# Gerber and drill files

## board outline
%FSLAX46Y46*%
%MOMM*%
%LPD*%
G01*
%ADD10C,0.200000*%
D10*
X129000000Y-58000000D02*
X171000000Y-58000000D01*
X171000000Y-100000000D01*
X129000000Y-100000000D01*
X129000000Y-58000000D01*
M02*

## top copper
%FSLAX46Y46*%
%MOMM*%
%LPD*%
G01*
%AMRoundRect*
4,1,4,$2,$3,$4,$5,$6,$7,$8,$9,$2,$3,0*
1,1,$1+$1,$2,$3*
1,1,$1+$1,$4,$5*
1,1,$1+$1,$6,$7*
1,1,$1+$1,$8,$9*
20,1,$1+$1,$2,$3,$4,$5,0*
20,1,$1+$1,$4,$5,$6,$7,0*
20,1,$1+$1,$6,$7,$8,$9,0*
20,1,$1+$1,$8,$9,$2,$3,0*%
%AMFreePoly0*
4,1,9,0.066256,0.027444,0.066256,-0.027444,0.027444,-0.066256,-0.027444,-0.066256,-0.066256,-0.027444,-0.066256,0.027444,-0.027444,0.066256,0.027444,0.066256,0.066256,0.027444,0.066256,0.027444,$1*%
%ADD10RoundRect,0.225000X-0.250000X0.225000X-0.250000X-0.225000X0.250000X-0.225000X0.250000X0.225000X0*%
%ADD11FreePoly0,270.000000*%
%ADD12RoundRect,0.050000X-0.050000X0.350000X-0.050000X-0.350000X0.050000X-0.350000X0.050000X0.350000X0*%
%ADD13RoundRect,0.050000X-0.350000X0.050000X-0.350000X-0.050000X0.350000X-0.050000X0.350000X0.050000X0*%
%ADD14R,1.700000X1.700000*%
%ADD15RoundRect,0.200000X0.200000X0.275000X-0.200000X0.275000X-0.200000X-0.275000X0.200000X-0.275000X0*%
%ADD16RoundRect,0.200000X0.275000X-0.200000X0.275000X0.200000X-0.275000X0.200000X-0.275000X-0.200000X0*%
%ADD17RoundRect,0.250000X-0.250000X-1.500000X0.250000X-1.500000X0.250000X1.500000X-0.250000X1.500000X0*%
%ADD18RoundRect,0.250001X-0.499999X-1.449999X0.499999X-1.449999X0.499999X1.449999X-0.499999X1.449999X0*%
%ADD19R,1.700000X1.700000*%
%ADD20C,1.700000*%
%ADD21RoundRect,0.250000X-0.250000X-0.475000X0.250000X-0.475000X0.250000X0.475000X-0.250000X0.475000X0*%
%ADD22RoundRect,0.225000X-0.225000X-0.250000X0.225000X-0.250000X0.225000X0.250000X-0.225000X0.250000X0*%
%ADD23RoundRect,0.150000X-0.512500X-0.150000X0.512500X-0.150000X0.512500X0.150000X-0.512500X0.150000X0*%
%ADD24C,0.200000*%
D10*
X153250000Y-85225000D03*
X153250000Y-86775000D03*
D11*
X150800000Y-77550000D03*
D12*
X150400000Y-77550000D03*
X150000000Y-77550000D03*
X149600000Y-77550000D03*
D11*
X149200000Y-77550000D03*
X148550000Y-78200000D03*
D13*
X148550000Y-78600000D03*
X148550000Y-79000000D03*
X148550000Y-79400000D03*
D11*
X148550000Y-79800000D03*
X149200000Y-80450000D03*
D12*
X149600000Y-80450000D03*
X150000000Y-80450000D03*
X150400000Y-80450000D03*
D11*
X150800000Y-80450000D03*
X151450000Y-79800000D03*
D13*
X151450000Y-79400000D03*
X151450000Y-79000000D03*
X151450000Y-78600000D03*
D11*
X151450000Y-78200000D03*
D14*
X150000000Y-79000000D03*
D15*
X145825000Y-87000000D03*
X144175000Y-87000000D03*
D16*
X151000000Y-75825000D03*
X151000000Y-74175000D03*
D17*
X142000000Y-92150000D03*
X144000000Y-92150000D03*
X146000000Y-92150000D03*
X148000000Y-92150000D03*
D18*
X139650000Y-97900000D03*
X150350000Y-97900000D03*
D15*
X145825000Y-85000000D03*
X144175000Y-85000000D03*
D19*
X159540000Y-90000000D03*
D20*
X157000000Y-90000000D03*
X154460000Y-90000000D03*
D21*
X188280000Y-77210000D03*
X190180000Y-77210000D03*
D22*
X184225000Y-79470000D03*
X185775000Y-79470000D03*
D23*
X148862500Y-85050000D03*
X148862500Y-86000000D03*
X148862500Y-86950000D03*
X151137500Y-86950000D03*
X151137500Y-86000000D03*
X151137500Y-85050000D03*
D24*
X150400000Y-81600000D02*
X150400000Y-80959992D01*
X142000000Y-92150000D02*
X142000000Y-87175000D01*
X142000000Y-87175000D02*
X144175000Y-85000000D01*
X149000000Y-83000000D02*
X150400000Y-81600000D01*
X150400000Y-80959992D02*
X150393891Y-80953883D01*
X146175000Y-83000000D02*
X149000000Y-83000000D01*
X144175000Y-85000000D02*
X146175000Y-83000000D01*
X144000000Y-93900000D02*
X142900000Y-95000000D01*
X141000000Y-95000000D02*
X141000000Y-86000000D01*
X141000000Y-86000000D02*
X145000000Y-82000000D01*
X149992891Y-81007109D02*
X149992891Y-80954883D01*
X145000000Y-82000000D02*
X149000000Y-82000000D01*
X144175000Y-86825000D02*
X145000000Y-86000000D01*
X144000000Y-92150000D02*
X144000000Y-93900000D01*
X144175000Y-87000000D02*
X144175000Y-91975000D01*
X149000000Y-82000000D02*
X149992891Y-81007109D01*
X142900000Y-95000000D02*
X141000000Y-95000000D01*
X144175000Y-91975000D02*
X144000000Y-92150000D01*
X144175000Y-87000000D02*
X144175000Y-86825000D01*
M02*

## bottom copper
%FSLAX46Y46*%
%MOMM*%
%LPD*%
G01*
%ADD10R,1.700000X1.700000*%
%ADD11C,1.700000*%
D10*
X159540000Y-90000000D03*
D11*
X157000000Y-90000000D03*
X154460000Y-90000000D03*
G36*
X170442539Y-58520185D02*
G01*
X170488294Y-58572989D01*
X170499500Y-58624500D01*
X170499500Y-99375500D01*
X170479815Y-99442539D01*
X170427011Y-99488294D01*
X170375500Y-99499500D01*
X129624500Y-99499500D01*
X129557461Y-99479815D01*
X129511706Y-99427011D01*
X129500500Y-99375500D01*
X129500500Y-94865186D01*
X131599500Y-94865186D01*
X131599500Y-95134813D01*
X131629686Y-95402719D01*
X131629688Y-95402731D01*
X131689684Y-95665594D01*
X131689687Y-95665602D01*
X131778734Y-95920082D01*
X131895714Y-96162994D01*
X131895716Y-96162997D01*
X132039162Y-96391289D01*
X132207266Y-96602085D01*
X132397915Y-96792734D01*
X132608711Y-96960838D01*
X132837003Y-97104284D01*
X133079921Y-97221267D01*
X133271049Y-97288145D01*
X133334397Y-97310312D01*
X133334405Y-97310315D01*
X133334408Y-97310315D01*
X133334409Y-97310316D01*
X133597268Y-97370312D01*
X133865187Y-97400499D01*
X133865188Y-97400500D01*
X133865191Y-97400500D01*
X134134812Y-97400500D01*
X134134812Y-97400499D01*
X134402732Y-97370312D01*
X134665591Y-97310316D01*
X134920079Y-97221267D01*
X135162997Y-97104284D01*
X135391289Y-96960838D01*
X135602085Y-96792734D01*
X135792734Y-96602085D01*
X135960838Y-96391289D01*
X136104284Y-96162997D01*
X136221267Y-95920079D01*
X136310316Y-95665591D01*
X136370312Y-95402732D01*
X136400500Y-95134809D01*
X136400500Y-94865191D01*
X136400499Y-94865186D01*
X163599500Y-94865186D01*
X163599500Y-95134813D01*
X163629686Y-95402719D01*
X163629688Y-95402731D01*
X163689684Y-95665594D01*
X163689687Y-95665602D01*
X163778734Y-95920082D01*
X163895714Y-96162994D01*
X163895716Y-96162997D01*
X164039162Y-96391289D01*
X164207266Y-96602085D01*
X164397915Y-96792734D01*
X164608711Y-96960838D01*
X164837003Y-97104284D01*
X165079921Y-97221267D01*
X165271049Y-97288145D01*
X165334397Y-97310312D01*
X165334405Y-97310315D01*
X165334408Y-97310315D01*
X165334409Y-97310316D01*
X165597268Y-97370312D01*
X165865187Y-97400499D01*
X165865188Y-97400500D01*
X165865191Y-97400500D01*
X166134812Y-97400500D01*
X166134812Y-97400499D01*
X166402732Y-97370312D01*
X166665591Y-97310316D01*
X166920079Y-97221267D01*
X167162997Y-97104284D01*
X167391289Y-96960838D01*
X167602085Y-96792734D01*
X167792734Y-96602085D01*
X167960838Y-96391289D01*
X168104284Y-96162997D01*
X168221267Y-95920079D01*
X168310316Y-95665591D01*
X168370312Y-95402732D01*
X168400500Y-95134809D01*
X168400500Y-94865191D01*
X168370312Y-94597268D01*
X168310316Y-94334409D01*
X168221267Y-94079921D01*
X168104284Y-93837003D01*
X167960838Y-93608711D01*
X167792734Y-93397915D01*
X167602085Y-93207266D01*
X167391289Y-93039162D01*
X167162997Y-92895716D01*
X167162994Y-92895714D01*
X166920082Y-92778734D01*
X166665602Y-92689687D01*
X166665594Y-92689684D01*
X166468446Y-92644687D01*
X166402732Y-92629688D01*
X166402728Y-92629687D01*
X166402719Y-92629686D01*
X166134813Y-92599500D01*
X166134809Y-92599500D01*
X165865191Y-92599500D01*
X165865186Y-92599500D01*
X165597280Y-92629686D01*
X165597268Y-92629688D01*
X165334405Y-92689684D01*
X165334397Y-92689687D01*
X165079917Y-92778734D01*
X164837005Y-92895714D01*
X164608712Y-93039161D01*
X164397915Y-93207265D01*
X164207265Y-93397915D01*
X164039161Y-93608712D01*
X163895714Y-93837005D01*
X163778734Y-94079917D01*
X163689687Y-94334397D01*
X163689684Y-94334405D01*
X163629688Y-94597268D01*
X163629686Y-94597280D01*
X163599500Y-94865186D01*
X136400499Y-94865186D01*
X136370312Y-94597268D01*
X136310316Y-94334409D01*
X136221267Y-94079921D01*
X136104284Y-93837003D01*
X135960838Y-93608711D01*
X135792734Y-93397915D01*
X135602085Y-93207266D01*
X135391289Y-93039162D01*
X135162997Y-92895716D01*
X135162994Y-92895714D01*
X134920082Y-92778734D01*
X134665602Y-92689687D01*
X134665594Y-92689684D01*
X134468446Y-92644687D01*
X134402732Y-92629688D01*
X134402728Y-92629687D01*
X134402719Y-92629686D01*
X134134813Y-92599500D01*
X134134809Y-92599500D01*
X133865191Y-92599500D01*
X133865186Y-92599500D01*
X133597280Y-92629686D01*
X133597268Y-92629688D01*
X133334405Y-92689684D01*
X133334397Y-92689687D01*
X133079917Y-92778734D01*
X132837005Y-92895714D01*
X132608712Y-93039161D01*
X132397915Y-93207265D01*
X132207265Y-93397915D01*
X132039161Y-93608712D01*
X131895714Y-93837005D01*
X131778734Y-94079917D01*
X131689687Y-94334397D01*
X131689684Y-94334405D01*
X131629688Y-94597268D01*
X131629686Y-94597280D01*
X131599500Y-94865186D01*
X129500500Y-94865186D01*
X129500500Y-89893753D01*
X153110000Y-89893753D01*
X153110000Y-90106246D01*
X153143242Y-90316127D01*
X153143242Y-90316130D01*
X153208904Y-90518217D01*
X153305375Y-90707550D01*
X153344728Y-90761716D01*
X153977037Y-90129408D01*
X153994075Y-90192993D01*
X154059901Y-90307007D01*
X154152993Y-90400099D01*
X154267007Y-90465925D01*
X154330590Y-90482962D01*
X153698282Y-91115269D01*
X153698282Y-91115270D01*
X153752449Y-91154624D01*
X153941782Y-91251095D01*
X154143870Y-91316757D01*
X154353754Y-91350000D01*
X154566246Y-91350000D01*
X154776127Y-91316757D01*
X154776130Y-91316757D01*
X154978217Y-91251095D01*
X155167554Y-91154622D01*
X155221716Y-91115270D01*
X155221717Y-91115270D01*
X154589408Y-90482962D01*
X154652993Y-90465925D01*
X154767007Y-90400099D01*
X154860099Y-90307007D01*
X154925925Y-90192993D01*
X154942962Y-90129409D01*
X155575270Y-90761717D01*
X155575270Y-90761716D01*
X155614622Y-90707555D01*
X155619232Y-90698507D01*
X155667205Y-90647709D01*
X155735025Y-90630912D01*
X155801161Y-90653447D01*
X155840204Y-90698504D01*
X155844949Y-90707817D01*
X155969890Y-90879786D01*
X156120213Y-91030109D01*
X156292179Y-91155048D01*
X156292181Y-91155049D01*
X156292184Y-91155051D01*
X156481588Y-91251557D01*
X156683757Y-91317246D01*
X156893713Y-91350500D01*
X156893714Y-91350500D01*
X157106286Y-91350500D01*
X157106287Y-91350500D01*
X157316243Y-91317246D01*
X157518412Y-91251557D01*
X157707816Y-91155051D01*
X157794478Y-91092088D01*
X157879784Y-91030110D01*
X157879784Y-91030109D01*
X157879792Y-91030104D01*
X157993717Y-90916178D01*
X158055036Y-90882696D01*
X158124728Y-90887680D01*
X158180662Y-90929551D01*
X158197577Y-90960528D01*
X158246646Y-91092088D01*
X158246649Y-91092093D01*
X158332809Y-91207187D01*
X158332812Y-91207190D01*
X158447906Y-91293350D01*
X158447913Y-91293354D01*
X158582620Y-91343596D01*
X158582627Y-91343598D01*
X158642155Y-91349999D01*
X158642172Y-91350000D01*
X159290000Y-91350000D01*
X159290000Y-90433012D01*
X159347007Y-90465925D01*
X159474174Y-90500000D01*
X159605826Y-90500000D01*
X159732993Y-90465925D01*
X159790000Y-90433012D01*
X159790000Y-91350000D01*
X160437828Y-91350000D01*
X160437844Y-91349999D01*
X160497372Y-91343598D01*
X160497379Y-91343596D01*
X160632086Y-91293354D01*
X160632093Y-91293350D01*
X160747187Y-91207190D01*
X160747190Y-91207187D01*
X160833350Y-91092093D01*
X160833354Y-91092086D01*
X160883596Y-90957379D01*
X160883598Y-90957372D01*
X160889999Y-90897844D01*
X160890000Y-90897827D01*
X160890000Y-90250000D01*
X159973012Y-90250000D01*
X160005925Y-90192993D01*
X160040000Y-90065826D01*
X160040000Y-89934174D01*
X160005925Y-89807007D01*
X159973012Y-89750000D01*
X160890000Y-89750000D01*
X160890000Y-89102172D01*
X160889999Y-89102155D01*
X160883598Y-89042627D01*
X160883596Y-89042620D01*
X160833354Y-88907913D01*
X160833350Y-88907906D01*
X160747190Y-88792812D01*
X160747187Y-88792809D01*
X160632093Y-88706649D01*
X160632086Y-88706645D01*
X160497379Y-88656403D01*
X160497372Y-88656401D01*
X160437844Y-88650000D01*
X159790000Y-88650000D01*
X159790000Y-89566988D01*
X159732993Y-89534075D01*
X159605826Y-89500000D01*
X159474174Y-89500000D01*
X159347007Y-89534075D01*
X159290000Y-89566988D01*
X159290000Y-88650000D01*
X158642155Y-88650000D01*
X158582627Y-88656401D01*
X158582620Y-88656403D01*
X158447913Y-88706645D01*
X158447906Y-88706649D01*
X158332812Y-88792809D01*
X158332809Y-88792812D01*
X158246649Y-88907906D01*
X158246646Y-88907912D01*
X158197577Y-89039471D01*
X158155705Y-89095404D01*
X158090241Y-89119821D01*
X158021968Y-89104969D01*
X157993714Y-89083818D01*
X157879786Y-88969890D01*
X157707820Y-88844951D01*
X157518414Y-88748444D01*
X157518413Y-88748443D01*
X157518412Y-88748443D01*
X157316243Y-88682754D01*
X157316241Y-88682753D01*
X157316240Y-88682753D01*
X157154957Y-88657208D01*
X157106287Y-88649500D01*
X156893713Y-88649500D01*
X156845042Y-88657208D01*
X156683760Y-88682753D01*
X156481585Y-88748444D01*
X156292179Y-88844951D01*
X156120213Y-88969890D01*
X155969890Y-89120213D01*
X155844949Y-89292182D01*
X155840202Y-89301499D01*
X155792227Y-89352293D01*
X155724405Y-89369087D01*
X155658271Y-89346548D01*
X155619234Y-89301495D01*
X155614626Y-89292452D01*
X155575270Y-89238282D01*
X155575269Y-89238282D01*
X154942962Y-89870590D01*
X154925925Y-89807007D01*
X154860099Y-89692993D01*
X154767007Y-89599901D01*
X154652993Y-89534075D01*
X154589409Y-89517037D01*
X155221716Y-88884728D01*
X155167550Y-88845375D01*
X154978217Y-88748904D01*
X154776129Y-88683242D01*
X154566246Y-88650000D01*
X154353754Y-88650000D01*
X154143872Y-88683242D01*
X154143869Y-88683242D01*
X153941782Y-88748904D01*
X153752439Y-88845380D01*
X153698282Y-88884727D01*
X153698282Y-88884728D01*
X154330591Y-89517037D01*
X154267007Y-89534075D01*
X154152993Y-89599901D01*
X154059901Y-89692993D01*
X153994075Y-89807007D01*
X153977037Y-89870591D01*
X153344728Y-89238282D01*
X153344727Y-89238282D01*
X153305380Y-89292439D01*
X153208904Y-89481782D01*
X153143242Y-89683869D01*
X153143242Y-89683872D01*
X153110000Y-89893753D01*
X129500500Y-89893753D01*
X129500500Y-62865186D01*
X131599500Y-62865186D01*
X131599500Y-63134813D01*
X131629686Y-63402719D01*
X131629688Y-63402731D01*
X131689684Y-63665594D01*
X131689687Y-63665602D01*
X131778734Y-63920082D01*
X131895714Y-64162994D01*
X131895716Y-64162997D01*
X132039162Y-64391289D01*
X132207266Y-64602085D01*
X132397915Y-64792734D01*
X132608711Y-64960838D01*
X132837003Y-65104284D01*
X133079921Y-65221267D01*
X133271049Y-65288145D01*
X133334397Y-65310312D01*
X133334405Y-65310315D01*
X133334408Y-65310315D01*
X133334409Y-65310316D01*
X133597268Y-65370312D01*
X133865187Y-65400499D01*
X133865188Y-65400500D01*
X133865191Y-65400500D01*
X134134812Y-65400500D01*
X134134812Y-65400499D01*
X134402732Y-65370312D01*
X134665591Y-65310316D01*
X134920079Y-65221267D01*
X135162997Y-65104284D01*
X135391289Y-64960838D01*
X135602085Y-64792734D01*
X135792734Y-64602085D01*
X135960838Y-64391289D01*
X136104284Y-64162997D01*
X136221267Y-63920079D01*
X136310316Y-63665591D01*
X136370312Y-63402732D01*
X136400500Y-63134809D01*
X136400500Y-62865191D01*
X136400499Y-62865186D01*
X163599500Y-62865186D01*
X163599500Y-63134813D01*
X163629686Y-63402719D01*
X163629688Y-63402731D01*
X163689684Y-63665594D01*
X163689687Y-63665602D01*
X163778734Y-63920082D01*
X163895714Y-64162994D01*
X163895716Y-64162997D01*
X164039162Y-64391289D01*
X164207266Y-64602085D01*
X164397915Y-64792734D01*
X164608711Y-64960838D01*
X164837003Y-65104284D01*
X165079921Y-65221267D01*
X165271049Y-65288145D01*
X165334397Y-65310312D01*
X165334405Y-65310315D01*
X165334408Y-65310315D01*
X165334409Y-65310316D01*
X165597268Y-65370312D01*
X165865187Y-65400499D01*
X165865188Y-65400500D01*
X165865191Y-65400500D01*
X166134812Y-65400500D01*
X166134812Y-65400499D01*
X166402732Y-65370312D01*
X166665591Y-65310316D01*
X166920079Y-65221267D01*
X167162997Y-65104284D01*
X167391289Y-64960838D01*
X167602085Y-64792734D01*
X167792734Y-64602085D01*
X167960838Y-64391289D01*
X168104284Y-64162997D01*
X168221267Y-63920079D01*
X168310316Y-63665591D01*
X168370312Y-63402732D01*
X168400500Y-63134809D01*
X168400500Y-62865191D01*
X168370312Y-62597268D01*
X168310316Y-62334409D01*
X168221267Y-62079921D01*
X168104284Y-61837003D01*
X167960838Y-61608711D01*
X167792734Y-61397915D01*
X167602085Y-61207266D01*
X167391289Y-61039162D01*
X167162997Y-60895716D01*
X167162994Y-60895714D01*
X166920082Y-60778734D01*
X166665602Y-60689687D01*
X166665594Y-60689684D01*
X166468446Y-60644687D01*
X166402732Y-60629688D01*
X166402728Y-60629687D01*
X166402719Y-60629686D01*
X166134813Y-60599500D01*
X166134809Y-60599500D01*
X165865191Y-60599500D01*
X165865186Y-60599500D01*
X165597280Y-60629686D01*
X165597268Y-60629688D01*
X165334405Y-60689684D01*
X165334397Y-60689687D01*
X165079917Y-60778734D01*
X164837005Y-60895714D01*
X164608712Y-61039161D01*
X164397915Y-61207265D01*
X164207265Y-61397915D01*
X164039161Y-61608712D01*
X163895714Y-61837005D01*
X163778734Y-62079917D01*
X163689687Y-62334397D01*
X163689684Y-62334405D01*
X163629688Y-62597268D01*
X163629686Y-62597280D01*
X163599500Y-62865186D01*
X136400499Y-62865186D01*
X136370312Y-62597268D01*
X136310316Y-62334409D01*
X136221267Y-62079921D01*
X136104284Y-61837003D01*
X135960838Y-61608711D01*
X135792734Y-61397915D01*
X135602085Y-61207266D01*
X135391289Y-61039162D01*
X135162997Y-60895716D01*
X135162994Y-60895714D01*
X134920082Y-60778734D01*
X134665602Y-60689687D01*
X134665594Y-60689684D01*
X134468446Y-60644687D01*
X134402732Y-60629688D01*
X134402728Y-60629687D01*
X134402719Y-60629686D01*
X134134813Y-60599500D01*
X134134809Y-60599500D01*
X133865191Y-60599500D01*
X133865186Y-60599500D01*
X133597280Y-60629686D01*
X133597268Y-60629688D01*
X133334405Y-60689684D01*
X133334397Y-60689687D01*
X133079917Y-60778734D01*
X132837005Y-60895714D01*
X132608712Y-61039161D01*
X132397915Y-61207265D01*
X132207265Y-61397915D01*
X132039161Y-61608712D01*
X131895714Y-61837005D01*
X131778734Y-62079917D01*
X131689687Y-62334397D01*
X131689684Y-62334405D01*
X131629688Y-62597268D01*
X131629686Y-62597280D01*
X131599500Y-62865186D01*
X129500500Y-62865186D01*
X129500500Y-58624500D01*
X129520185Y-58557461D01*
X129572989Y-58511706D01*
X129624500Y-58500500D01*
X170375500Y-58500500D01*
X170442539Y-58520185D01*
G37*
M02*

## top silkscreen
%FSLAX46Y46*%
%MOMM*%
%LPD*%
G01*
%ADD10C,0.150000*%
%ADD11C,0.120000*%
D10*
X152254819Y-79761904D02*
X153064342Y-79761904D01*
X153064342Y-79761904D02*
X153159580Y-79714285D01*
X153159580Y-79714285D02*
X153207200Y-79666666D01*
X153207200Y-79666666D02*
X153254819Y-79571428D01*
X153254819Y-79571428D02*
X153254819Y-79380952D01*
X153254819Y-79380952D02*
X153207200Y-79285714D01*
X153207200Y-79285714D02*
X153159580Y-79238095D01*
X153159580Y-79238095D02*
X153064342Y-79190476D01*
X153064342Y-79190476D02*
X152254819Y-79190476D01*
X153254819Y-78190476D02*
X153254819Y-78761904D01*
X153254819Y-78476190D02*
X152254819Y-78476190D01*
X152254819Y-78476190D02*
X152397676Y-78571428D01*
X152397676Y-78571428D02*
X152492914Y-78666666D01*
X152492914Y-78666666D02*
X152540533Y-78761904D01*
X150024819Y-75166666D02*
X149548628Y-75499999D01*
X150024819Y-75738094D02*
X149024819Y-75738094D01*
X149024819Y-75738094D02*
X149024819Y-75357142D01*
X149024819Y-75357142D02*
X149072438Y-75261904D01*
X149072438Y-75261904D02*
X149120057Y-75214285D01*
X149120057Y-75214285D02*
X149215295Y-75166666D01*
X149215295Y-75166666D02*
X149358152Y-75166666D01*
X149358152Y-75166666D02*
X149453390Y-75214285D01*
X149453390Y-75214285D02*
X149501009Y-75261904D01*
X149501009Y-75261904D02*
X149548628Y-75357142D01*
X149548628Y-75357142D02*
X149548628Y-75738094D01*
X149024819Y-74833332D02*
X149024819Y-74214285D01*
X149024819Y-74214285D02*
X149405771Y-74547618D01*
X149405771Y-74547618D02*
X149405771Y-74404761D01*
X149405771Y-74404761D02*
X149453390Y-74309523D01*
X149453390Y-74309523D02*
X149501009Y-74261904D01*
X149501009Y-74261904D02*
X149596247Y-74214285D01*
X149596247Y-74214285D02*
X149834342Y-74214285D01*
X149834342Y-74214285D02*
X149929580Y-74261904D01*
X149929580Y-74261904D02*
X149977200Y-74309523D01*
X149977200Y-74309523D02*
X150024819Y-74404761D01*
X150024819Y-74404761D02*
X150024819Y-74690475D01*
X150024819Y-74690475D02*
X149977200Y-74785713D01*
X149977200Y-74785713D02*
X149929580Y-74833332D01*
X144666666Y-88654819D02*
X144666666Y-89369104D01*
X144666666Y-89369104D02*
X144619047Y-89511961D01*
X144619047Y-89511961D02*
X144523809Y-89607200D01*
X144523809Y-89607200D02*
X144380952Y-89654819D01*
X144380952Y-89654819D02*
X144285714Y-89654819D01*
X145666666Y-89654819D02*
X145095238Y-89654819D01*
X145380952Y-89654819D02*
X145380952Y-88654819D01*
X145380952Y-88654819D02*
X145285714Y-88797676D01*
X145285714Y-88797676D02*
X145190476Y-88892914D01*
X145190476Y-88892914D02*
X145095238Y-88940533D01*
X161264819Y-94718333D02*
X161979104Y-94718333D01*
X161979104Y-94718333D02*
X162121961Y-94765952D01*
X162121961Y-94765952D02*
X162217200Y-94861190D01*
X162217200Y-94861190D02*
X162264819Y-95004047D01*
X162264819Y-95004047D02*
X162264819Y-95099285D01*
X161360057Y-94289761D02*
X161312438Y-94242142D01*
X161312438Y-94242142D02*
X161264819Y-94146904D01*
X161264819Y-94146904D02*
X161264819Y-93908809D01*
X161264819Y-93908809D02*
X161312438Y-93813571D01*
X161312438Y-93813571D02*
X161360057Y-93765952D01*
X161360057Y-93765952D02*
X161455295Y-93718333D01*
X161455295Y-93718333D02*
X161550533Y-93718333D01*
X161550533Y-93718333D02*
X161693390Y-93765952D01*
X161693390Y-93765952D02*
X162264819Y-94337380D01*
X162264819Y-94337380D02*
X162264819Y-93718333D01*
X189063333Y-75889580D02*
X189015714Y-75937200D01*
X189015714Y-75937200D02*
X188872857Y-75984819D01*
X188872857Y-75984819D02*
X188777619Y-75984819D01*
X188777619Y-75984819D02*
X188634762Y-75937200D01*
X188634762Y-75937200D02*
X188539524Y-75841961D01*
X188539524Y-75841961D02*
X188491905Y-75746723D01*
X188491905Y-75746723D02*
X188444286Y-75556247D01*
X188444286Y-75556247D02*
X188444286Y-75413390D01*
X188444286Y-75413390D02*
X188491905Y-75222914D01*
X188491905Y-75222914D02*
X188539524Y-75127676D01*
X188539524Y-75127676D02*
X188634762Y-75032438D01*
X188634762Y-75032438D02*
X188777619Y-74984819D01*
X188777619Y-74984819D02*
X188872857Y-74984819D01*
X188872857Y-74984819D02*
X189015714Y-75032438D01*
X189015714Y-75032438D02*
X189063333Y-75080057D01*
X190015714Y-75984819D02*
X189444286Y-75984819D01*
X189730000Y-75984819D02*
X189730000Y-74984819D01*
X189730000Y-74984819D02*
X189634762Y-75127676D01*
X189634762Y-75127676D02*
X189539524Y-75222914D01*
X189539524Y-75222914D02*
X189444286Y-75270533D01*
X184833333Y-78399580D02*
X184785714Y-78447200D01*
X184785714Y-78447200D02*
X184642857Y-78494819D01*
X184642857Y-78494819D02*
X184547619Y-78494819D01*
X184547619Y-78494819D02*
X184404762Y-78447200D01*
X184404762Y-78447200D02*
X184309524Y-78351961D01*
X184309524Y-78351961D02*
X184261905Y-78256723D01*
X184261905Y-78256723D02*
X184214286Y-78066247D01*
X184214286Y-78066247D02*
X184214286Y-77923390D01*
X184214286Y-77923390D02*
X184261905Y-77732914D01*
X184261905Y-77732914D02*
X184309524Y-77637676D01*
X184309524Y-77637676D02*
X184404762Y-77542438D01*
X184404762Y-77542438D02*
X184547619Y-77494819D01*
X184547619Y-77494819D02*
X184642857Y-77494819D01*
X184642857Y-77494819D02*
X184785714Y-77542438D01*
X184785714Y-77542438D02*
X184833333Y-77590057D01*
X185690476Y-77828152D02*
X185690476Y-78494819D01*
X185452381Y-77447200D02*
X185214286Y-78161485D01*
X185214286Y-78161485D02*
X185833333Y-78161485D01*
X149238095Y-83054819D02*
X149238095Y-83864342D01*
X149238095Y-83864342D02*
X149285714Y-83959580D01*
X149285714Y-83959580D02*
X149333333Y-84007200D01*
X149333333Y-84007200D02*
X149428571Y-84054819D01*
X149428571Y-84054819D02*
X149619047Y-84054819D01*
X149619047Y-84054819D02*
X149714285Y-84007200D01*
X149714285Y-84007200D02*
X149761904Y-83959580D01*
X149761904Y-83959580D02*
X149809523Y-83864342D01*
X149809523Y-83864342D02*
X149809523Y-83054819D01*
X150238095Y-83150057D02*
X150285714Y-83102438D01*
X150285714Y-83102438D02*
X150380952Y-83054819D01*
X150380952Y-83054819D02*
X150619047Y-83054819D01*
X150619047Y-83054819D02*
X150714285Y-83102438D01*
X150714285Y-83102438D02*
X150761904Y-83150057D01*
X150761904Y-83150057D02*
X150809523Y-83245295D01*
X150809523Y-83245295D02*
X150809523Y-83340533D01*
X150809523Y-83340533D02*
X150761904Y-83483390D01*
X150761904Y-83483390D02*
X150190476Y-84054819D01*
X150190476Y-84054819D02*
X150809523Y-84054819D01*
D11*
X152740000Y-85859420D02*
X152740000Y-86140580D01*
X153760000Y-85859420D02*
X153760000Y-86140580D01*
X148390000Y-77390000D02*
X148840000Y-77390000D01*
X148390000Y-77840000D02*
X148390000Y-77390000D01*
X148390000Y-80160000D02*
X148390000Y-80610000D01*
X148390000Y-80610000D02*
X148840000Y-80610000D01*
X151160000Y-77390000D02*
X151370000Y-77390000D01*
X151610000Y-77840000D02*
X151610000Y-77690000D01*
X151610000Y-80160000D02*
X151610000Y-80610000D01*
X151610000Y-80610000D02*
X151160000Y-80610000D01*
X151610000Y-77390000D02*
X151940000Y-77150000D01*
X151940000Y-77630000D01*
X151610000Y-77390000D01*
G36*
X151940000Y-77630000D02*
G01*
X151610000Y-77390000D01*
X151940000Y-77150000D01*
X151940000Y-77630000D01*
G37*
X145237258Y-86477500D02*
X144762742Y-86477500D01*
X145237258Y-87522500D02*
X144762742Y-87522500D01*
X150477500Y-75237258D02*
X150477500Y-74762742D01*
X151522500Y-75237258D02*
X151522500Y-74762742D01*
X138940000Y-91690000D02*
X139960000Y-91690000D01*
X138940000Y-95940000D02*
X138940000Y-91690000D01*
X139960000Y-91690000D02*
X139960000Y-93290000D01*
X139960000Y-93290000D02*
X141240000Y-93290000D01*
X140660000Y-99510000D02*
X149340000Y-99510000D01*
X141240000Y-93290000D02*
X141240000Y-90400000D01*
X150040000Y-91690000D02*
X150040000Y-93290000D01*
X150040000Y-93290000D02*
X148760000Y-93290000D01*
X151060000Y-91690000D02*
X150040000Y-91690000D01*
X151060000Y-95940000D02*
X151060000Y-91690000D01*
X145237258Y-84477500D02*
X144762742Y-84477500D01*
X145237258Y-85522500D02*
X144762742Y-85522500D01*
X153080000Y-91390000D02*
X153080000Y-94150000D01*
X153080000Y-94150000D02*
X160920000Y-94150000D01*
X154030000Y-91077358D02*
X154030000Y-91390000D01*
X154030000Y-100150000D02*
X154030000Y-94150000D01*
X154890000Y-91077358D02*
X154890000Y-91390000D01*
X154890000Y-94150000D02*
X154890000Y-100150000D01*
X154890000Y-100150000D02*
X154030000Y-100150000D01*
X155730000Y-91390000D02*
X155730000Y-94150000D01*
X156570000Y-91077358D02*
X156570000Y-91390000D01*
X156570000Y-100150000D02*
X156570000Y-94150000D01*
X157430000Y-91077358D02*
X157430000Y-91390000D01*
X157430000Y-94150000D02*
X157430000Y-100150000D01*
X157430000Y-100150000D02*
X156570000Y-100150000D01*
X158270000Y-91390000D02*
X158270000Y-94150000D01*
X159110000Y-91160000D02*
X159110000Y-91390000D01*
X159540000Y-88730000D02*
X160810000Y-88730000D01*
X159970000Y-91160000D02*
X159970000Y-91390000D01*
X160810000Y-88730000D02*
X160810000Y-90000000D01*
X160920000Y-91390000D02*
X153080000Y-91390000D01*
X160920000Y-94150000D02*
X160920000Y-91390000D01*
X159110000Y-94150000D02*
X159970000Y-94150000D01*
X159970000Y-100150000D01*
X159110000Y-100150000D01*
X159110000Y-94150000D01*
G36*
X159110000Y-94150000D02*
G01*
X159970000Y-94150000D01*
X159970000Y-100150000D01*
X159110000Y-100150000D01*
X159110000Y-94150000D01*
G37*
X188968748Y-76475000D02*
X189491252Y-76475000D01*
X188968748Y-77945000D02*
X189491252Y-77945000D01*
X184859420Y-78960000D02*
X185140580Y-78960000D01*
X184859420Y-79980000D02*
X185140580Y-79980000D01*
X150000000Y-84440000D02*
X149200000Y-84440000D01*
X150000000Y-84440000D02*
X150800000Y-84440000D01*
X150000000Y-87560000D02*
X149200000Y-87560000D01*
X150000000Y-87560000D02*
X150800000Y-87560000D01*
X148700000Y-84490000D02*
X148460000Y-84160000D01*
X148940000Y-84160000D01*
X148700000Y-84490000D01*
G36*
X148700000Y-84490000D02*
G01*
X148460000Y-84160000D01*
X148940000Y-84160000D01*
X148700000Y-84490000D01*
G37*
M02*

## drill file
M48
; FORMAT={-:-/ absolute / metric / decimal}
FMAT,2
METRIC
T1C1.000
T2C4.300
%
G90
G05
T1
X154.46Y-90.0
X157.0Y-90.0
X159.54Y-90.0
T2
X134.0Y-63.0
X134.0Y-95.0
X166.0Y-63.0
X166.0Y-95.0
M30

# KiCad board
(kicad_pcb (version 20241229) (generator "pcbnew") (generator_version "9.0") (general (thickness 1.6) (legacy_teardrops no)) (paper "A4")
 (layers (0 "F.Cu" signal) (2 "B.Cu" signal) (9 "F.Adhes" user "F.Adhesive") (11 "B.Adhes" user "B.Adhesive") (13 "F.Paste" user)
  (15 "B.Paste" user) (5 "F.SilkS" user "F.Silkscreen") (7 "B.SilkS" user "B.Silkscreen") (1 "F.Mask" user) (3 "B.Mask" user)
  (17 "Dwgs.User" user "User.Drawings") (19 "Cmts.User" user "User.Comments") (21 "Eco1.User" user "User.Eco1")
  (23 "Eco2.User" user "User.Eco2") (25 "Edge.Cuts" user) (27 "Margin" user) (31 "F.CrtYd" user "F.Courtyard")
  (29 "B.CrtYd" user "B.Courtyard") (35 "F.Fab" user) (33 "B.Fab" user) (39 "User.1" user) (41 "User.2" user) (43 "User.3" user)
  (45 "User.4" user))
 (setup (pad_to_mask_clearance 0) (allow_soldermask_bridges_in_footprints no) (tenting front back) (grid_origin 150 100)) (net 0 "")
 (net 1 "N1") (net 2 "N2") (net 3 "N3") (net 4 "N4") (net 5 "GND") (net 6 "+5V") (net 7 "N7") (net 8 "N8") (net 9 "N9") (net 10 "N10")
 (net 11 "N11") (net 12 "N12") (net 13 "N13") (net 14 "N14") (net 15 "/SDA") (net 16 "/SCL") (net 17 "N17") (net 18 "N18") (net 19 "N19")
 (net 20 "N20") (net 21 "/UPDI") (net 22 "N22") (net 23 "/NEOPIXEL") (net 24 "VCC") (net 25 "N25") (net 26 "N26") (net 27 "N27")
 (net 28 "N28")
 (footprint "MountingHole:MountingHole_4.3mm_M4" (layer "F.Cu") (at 134 63)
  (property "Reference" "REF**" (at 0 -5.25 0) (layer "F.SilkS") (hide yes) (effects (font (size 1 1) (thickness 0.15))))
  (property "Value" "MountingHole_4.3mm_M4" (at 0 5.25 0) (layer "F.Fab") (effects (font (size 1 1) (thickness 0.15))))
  (pad "" np_thru_hole circle (at 0 0) (size 4.3 4.3) (drill 4.3) (layers "*.Cu" "*.Mask")))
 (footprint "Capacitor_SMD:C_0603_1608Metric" (layer "F.Cu") (at 153.25 86 -90)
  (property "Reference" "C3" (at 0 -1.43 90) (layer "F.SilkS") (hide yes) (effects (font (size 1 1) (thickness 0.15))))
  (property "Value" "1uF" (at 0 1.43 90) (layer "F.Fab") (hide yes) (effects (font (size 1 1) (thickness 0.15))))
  (fp_line (start -0.14058 0.51) (end 0.14058 0.51) (stroke (width 0.12) (type solid)) (layer "F.SilkS"))
  (fp_line (start -0.14058 -0.51) (end 0.14058 -0.51) (stroke (width 0.12) (type solid)) (layer "F.SilkS"))
  (pad "1" smd roundrect (at -0.775 0 270) (size 0.9 0.95) (layers "F.Cu" "F.Mask" "F.Paste") (roundrect_rratio 0.25) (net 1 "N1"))
  (pad "2" smd roundrect (at 0.775 0 270) (size 0.9 0.95) (layers "F.Cu" "F.Mask" "F.Paste") (roundrect_rratio 0.25) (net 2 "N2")))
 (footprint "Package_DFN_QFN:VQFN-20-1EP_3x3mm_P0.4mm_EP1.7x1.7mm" (layer "F.Cu") (at 150 79 -90)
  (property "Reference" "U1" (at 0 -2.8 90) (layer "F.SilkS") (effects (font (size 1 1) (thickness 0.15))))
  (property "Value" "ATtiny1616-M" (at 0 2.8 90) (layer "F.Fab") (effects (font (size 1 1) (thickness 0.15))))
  (fp_line (start -1.61 1.61) (end -1.61 1.16) (stroke (width 0.12) (type solid)) (layer "F.SilkS"))
  (fp_line (start -1.16 1.61) (end -1.61 1.61) (stroke (width 0.12) (type solid)) (layer "F.SilkS"))
  (fp_line (start 1.16 1.61) (end 1.61 1.61) (stroke (width 0.12) (type solid)) (layer "F.SilkS"))
  (fp_line (start 1.61 1.61) (end 1.61 1.16) (stroke (width 0.12) (type solid)) (layer "F.SilkS"))
  (fp_line (start -1.61 -1.16) (end -1.61 -1.37) (stroke (width 0.12) (type solid)) (layer "F.SilkS"))
  (fp_line (start -1.16 -1.61) (end -1.31 -1.61) (stroke (width 0.12) (type solid)) (layer "F.SilkS"))
  (fp_line (start 1.16 -1.61) (end 1.61 -1.61) (stroke (width 0.12) (type solid)) (layer "F.SilkS"))
  (fp_line (start 1.61 -1.61) (end 1.61 -1.16) (stroke (width 0.12) (type solid)) (layer "F.SilkS"))
  (fp_poly (pts (xy -1.61 -1.61) (xy -1.85 -1.94) (xy -1.37 -1.94)) (stroke (width 0.12) (type solid)) (fill yes) (layer "F.SilkS"))
  (pad "" smd roundrect (at -0.425 -0.425 270) (size 0.69 0.69) (layers "F.Paste") (roundrect_rratio 0.25))
  (pad "" smd roundrect (at -0.425 0.425 270) (size 0.69 0.69) (layers "F.Paste") (roundrect_rratio 0.25))
  (pad "" smd roundrect (at 0.425 -0.425 270) (size 0.69 0.69) (layers "F.Paste") (roundrect_rratio 0.25))
  (pad "" smd roundrect (at 0.425 0.425 270) (size 0.69 0.69) (layers "F.Paste") (roundrect_rratio 0.25))
  (pad "1" smd custom (at -1.45 -0.8 270) (size 0.143431 0.143431) (layers "F.Cu" "F.Mask" "F.Paste") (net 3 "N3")
   (options (clearance outline) (anchor circle)) (primitives))
  (pad "2" smd roundrect (at -1.45 -0.4 270) (size 0.8 0.2) (layers "F.Cu" "F.Mask" "F.Paste") (roundrect_rratio 0.25) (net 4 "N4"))
  (pad "3" smd roundrect (at -1.45 0 270) (size 0.8 0.2) (layers "F.Cu" "F.Mask" "F.Paste") (roundrect_rratio 0.25) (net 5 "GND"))
  (pad "4" smd roundrect (at -1.45 0.4 270) (size 0.8 0.2) (layers "F.Cu" "F.Mask" "F.Paste") (roundrect_rratio 0.25) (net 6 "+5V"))
  (pad "5" smd custom (at -1.45 0.8 270) (size 0.143431 0.143431) (layers "F.Cu" "F.Mask" "F.Paste") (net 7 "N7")
   (options (clearance outline) (anchor circle)) (primitives))
  (pad "6" smd custom (at -0.8 1.45 270) (size 0.143431 0.143431) (layers "F.Cu" "F.Mask" "F.Paste") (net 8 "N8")
   (options (clearance outline) (anchor circle)) (primitives))
  (pad "7" smd roundrect (at -0.4 1.45 270) (size 0.2 0.8) (layers "F.Cu" "F.Mask" "F.Paste") (roundrect_rratio 0.25) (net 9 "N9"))
  (pad "8" smd roundrect (at 0 1.45 270) (size 0.2 0.8) (layers "F.Cu" "F.Mask" "F.Paste") (roundrect_rratio 0.25) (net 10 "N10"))
  (pad "9" smd roundrect (at 0.4 1.45 270) (size 0.2 0.8) (layers "F.Cu" "F.Mask" "F.Paste") (roundrect_rratio 0.25) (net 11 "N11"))
  (pad "10" smd custom (at 0.8 1.45 270) (size 0.143431 0.143431) (layers "F.Cu" "F.Mask" "F.Paste") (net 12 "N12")
   (options (clearance outline) (anchor circle)) (primitives))
  (pad "11" smd custom (at 1.45 0.8 270) (size 0.143431 0.143431) (layers "F.Cu" "F.Mask" "F.Paste") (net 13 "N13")
   (options (clearance outline) (anchor circle)) (primitives))
  (pad "12" smd roundrect (at 1.45 0.4 270) (size 0.8 0.2) (layers "F.Cu" "F.Mask" "F.Paste") (roundrect_rratio 0.25) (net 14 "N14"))
  (pad "13" smd roundrect (at 1.45 0 270) (size 0.8 0.2) (layers "F.Cu" "F.Mask" "F.Paste") (roundrect_rratio 0.25) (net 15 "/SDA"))
  (pad "14" smd roundrect (at 1.45 -0.4 270) (size 0.8 0.2) (layers "F.Cu" "F.Mask" "F.Paste") (roundrect_rratio 0.25) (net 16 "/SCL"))
  (pad "15" smd custom (at 1.45 -0.8 270) (size 0.143431 0.143431) (layers "F.Cu" "F.Mask" "F.Paste") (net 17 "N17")
   (options (clearance outline) (anchor circle)) (primitives))
  (pad "16" smd custom (at 0.8 -1.45 270) (size 0.143431 0.143431) (layers "F.Cu" "F.Mask" "F.Paste") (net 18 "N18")
   (options (clearance outline) (anchor circle)) (primitives))
  (pad "17" smd roundrect (at 0.4 -1.45 270) (size 0.2 0.8) (layers "F.Cu" "F.Mask" "F.Paste") (roundrect_rratio 0.25) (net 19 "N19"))
  (pad "18" smd roundrect (at 0 -1.45 270) (size 0.2 0.8) (layers "F.Cu" "F.Mask" "F.Paste") (roundrect_rratio 0.25) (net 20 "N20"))
  (pad "19" smd roundrect (at -0.4 -1.45 270) (size 0.2 0.8) (layers "F.Cu" "F.Mask" "F.Paste") (roundrect_rratio 0.25) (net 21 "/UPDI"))
  (pad "20" smd custom (at -0.8 -1.45 270) (size 0.143431 0.143431) (layers "F.Cu" "F.Mask" "F.Paste") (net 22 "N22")
   (options (clearance outline) (anchor circle)) (primitives))
  (pad "21" smd rect (at 0 0 270) (size 1.7 1.7) (layers "F.Cu" "F.Mask") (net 5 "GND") (zone_connect 2)))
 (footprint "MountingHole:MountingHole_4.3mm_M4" (layer "F.Cu") (at 166 63)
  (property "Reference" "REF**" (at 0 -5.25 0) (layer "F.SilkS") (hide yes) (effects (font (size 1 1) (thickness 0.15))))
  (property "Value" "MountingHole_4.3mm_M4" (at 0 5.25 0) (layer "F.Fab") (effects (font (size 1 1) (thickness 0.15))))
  (pad "" np_thru_hole circle (at 0 0) (size 4.3 4.3) (drill 4.3) (layers "*.Cu" "*.Mask")))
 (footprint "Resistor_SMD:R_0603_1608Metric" (layer "F.Cu") (at 145 87 180)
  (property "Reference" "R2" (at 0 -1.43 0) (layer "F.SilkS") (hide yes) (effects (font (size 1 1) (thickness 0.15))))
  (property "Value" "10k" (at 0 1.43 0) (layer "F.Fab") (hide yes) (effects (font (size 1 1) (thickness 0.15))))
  (fp_line (start -0.237258 0.5225) (end 0.237258 0.5225) (stroke (width 0.12) (type solid)) (layer "F.SilkS"))
  (fp_line (start -0.237258 -0.5225) (end 0.237258 -0.5225) (stroke (width 0.12) (type solid)) (layer "F.SilkS"))
  (pad "1" smd roundrect (at -0.825 0 180) (size 0.8 0.95) (layers "F.Cu" "F.Mask" "F.Paste") (roundrect_rratio 0.25) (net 6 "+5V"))
  (pad "2" smd roundrect (at 0.825 0 180) (size 0.8 0.95) (layers "F.Cu" "F.Mask" "F.Paste") (roundrect_rratio 0.25) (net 15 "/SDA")))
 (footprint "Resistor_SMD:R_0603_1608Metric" (layer "F.Cu") (at 151 75 90)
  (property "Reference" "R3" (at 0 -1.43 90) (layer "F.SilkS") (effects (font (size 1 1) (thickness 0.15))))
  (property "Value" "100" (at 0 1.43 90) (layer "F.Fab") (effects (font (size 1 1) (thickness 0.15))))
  (fp_line (start -0.237258 -0.5225) (end 0.237258 -0.5225) (stroke (width 0.12) (type solid)) (layer "F.SilkS"))
  (fp_line (start -0.237258 0.5225) (end 0.237258 0.5225) (stroke (width 0.12) (type solid)) (layer "F.SilkS"))
  (pad "1" smd roundrect (at -0.825 0 90) (size 0.8 0.95) (layers "F.Cu" "F.Mask" "F.Paste") (roundrect_rratio 0.25) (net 3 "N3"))
  (pad "2" smd roundrect (at 0.825 0 90) (size 0.8 0.95) (layers "F.Cu" "F.Mask" "F.Paste") (roundrect_rratio 0.25) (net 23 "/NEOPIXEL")))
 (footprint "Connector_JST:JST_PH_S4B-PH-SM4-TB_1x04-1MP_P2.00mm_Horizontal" (layer "F.Cu") (at 145 95)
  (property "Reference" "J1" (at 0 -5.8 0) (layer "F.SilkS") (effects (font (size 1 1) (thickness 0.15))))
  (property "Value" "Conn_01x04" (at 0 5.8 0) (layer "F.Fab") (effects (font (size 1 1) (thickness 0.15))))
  (fp_line (start -6.06 -3.31) (end -5.04 -3.31) (stroke (width 0.12) (type solid)) (layer "F.SilkS"))
  (fp_line (start -6.06 0.94) (end -6.06 -3.31) (stroke (width 0.12) (type solid)) (layer "F.SilkS"))
  (fp_line (start -5.04 -3.31) (end -5.04 -1.71) (stroke (width 0.12) (type solid)) (layer "F.SilkS"))
  (fp_line (start -5.04 -1.71) (end -3.76 -1.71) (stroke (width 0.12) (type solid)) (layer "F.SilkS"))
  (fp_line (start -4.34 4.51) (end 4.34 4.51) (stroke (width 0.12) (type solid)) (layer "F.SilkS"))
  (fp_line (start -3.76 -1.71) (end -3.76 -4.6) (stroke (width 0.12) (type solid)) (layer "F.SilkS"))
  (fp_line (start 5.04 -3.31) (end 5.04 -1.71) (stroke (width 0.12) (type solid)) (layer "F.SilkS"))
  (fp_line (start 5.04 -1.71) (end 3.76 -1.71) (stroke (width 0.12) (type solid)) (layer "F.SilkS"))
  (fp_line (start 6.06 -3.31) (end 5.04 -3.31) (stroke (width 0.12) (type solid)) (layer "F.SilkS"))
  (fp_line (start 6.06 0.94) (end 6.06 -3.31) (stroke (width 0.12) (type solid)) (layer "F.SilkS"))
  (pad "1" smd roundrect (at -3 -2.85) (size 1 3.5) (layers "F.Cu" "F.Mask" "F.Paste") (roundrect_rratio 0.25) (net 16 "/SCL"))
  (pad "2" smd roundrect (at -1 -2.85) (size 1 3.5) (layers "F.Cu" "F.Mask" "F.Paste") (roundrect_rratio 0.25) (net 15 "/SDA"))
  (pad "3" smd roundrect (at 1 -2.85) (size 1 3.5) (layers "F.Cu" "F.Mask" "F.Paste") (roundrect_rratio 0.25) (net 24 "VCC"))
  (pad "4" smd roundrect (at 3 -2.85) (size 1 3.5) (layers "F.Cu" "F.Mask" "F.Paste") (roundrect_rratio 0.25) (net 5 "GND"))
  (pad "MP" smd roundrect (at -5.35 2.9) (size 1.5 3.4) (layers "F.Cu" "F.Mask" "F.Paste") (roundrect_rratio 0.166667))
  (pad "MP" smd roundrect (at 5.35 2.9) (size 1.5 3.4) (layers "F.Cu" "F.Mask" "F.Paste") (roundrect_rratio 0.166667)))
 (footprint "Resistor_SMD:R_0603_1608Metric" (layer "F.Cu") (at 145 85 180)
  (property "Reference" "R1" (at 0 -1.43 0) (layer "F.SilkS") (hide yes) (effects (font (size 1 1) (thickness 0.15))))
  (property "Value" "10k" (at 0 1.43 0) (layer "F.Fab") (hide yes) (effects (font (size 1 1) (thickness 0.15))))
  (fp_line (start -0.237258 0.5225) (end 0.237258 0.5225) (stroke (width 0.12) (type solid)) (layer "F.SilkS"))
  (fp_line (start -0.237258 -0.5225) (end 0.237258 -0.5225) (stroke (width 0.12) (type solid)) (layer "F.SilkS"))
  (pad "1" smd roundrect (at -0.825 0 180) (size 0.8 0.95) (layers "F.Cu" "F.Mask" "F.Paste") (roundrect_rratio 0.25) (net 6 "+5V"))
  (pad "2" smd roundrect (at 0.825 0 180) (size 0.8 0.95) (layers "F.Cu" "F.Mask" "F.Paste") (roundrect_rratio 0.25) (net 16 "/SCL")))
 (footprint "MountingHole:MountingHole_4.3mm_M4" (layer "F.Cu") (at 166 95)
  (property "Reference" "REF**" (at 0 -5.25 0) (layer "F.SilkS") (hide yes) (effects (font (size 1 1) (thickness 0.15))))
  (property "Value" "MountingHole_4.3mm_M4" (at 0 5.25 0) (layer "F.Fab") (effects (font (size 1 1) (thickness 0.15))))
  (pad "" np_thru_hole circle (at 0 0) (size 4.3 4.3) (drill 4.3) (layers "*.Cu" "*.Mask")))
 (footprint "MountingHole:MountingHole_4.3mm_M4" (layer "F.Cu") (at 134 95)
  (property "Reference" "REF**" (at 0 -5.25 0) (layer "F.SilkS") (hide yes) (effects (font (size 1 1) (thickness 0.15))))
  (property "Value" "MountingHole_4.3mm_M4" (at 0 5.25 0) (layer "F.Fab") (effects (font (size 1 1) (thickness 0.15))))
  (pad "" np_thru_hole circle (at 0 0) (size 4.3 4.3) (drill 4.3) (layers "*.Cu" "*.Mask")))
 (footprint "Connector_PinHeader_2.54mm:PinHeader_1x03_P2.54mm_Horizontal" (layer "F.Cu") (at 159.54 90 -90)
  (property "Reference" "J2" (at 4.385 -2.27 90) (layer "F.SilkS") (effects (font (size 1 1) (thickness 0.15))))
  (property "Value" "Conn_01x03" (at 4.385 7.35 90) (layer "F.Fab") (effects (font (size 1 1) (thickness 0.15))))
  (fp_line (start 1.39 6.46) (end 4.15 6.46) (stroke (width 0.12) (type solid)) (layer "F.SilkS"))
  (fp_line (start 4.15 6.46) (end 4.15 -1.38) (stroke (width 0.12) (type solid)) (layer "F.SilkS"))
  (fp_line (start 1.077358 5.51) (end 1.39 5.51) (stroke (width 0.12) (type solid)) (layer "F.SilkS"))
  (fp_line (start 10.15 5.51) (end 4.15 5.51) (stroke (width 0.12) (type solid)) (layer "F.SilkS"))
  (fp_line (start 1.077358 4.65) (end 1.39 4.65) (stroke (width 0.12) (type solid)) (layer "F.SilkS"))
  (fp_line (start 4.15 4.65) (end 10.15 4.65) (stroke (width 0.12) (type solid)) (layer "F.SilkS"))
  (fp_line (start 10.15 4.65) (end 10.15 5.51) (stroke (width 0.12) (type solid)) (layer "F.SilkS"))
  (fp_line (start 1.39 3.81) (end 4.15 3.81) (stroke (width 0.12) (type solid)) (layer "F.SilkS"))
  (fp_line (start 1.077358 2.97) (end 1.39 2.97) (stroke (width 0.12) (type solid)) (layer "F.SilkS"))
  (fp_line (start 10.15 2.97) (end 4.15 2.97) (stroke (width 0.12) (type solid)) (layer "F.SilkS"))
  (fp_line (start 1.077358 2.11) (end 1.39 2.11) (stroke (width 0.12) (type solid)) (layer "F.SilkS"))
  (fp_line (start 4.15 2.11) (end 10.15 2.11) (stroke (width 0.12) (type solid)) (layer "F.SilkS"))
  (fp_line (start 10.15 2.11) (end 10.15 2.97) (stroke (width 0.12) (type solid)) (layer "F.SilkS"))
  (fp_line (start 1.39 1.27) (end 4.15 1.27) (stroke (width 0.12) (type solid)) (layer "F.SilkS"))
  (fp_line (start 1.16 0.43) (end 1.39 0.43) (stroke (width 0.12) (type solid)) (layer "F.SilkS"))
  (fp_line (start -1.27 0) (end -1.27 -1.27) (stroke (width 0.12) (type solid)) (layer "F.SilkS"))
  (fp_line (start 1.16 -0.43) (end 1.39 -0.43) (stroke (width 0.12) (type solid)) (layer "F.SilkS"))
  (fp_line (start -1.27 -1.27) (end 0 -1.27) (stroke (width 0.12) (type solid)) (layer "F.SilkS"))
  (fp_line (start 1.39 -1.38) (end 1.39 6.46) (stroke (width 0.12) (type solid)) (layer "F.SilkS"))
  (fp_line (start 4.15 -1.38) (end 1.39 -1.38) (stroke (width 0.12) (type solid)) (layer "F.SilkS"))
  (fp_rect (start 4.15 -0.43) (end 10.15 0.43) (stroke (width 0.12) (type solid)) (fill yes) (layer "F.SilkS"))
  (pad "1" thru_hole rect (at 0 0 270) (size 1.7 1.7) (drill 1) (layers "*.Cu" "*.Mask") (remove_unused_layers no) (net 5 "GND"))
  (pad "2" thru_hole circle (at 0 2.54 270) (size 1.7 1.7) (drill 1) (layers "*.Cu" "*.Mask") (remove_unused_layers no) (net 6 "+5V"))
  (pad "3" thru_hole circle (at 0 5.08 270) (size 1.7 1.7) (drill 1) (layers "*.Cu" "*.Mask") (remove_unused_layers no) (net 5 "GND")))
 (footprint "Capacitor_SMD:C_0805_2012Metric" (layer "F.Cu") (at 189.23 77.21)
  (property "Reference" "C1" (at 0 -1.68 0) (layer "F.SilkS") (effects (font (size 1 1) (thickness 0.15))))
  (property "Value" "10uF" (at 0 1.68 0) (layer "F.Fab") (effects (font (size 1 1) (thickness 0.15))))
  (fp_line (start -0.261252 -0.735) (end 0.261252 -0.735) (stroke (width 0.12) (type solid)) (layer "F.SilkS"))
  (fp_line (start -0.261252 0.735) (end 0.261252 0.735) (stroke (width 0.12) (type solid)) (layer "F.SilkS"))
  (pad "1" smd roundrect (at -0.95 0) (size 1 1.45) (layers "F.Cu" "F.Mask" "F.Paste") (roundrect_rratio 0.25) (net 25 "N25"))
  (pad "2" smd roundrect (at 0.95 0) (size 1 1.45) (layers "F.Cu" "F.Mask" "F.Paste") (roundrect_rratio 0.25) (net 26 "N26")))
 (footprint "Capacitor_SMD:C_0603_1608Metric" (layer "F.Cu") (at 185 79.47)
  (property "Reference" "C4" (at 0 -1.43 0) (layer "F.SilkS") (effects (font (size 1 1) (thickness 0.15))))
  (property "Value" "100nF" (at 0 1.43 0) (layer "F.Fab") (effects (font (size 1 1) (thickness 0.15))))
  (fp_line (start -0.14058 -0.51) (end 0.14058 -0.51) (stroke (width 0.12) (type solid)) (layer "F.SilkS"))
  (fp_line (start -0.14058 0.51) (end 0.14058 0.51) (stroke (width 0.12) (type solid)) (layer "F.SilkS"))
  (pad "1" smd roundrect (at -0.775 0) (size 0.9 0.95) (layers "F.Cu" "F.Mask" "F.Paste") (roundrect_rratio 0.25) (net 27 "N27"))
  (pad "2" smd roundrect (at 0.775 0) (size 0.9 0.95) (layers "F.Cu" "F.Mask" "F.Paste") (roundrect_rratio 0.25) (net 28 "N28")))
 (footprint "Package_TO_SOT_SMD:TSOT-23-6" (layer "F.Cu") (at 150 86)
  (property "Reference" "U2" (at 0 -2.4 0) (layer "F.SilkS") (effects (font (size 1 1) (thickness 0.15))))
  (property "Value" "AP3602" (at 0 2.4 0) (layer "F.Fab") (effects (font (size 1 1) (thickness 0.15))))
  (fp_line (start 0 -1.56) (end -0.8 -1.56) (stroke (width 0.12) (type solid)) (layer "F.SilkS"))
  (fp_line (start 0 -1.56) (end 0.8 -1.56) (stroke (width 0.12) (type solid)) (layer "F.SilkS"))
  (fp_line (start 0 1.56) (end -0.8 1.56) (stroke (width 0.12) (type solid)) (layer "F.SilkS"))
  (fp_line (start 0 1.56) (end 0.8 1.56) (stroke (width 0.12) (type solid)) (layer "F.SilkS"))
  (fp_poly (pts (xy -1.3 -1.51) (xy -1.54 -1.84) (xy -1.06 -1.84)) (stroke (width 0.12) (type solid)) (fill yes) (layer "F.SilkS"))
  (pad "1" smd roundrect (at -1.1375 -0.95) (size 1.325 0.6) (layers "F.Cu" "F.Mask" "F.Paste") (roundrect_rratio 0.25) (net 6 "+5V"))
  (pad "2" smd roundrect (at -1.1375 0) (size 1.325 0.6) (layers "F.Cu" "F.Mask" "F.Paste") (roundrect_rratio 0.25) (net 5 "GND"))
  (pad "3" smd roundrect (at -1.1375 0.95) (size 1.325 0.6) (layers "F.Cu" "F.Mask" "F.Paste") (roundrect_rratio 0.25) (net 24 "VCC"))
  (pad "4" smd roundrect (at 1.1375 0.95) (size 1.325 0.6) (layers "F.Cu" "F.Mask" "F.Paste") (roundrect_rratio 0.25) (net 2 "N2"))
  (pad "5" smd roundrect (at 1.1375 0) (size 1.325 0.6) (layers "F.Cu" "F.Mask" "F.Paste") (roundrect_rratio 0.25) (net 24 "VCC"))
  (pad "6" smd roundrect (at 1.1375 -0.95) (size 1.325 0.6) (layers "F.Cu" "F.Mask" "F.Paste") (roundrect_rratio 0.25) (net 1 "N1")))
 (gr_rect (start 129 58) (end 171 100) (stroke (width 0.2) (type solid)) (fill no) (layer "Edge.Cuts"))
 (segment (start 150.4 81.6) (end 150.4 80.959992) (width 0.2) (layer "F.Cu") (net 16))
 (segment (start 142 92.15) (end 142 87.175) (width 0.2) (layer "F.Cu") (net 16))
 (segment (start 142 87.175) (end 144.175 85) (width 0.2) (layer "F.Cu") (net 16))
 (segment (start 149 83) (end 150.4 81.6) (width 0.2) (layer "F.Cu") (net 16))
 (segment (start 150.4 80.959992) (end 150.393891 80.953883) (width 0.2) (layer "F.Cu") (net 16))
 (segment (start 146.175 83) (end 149 83) (width 0.2) (layer "F.Cu") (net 16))
 (segment (start 144.175 85) (end 146.175 83) (width 0.2) (layer "F.Cu") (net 16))
 (segment (start 144 93.9) (end 142.9 95) (width 0.2) (layer "F.Cu") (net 15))
 (segment (start 141 95) (end 141 86) (width 0.2) (layer "F.Cu") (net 15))
 (segment (start 141 86) (end 145 82) (width 0.2) (layer "F.Cu") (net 15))
 (segment (start 149.992891 81.007109) (end 149.992891 80.954883) (width 0.2) (layer "F.Cu") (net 15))
 (segment (start 145 82) (end 149 82) (width 0.2) (layer "F.Cu") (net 15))
 (segment (start 144.175 86.825) (end 145 86) (width 0.2) (layer "F.Cu") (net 15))
 (segment (start 144 92.15) (end 144 93.9) (width 0.2) (layer "F.Cu") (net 15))
 (segment (start 144.175 87) (end 144.175 91.975) (width 0.2) (layer "F.Cu") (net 15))
 (segment (start 149 82) (end 149.992891 81.007109) (width 0.2) (layer "F.Cu") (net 15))
 (segment (start 142.9 95) (end 141 95) (width 0.2) (layer "F.Cu") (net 15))
 (segment (start 144.175 91.975) (end 144 92.15) (width 0.2) (layer "F.Cu") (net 15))
 (segment (start 144.175 87) (end 144.175 86.825) (width 0.2) (layer "F.Cu") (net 15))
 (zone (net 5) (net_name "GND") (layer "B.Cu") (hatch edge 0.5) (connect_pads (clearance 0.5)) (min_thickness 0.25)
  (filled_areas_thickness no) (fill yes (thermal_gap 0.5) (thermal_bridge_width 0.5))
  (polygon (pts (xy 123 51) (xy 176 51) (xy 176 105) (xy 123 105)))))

